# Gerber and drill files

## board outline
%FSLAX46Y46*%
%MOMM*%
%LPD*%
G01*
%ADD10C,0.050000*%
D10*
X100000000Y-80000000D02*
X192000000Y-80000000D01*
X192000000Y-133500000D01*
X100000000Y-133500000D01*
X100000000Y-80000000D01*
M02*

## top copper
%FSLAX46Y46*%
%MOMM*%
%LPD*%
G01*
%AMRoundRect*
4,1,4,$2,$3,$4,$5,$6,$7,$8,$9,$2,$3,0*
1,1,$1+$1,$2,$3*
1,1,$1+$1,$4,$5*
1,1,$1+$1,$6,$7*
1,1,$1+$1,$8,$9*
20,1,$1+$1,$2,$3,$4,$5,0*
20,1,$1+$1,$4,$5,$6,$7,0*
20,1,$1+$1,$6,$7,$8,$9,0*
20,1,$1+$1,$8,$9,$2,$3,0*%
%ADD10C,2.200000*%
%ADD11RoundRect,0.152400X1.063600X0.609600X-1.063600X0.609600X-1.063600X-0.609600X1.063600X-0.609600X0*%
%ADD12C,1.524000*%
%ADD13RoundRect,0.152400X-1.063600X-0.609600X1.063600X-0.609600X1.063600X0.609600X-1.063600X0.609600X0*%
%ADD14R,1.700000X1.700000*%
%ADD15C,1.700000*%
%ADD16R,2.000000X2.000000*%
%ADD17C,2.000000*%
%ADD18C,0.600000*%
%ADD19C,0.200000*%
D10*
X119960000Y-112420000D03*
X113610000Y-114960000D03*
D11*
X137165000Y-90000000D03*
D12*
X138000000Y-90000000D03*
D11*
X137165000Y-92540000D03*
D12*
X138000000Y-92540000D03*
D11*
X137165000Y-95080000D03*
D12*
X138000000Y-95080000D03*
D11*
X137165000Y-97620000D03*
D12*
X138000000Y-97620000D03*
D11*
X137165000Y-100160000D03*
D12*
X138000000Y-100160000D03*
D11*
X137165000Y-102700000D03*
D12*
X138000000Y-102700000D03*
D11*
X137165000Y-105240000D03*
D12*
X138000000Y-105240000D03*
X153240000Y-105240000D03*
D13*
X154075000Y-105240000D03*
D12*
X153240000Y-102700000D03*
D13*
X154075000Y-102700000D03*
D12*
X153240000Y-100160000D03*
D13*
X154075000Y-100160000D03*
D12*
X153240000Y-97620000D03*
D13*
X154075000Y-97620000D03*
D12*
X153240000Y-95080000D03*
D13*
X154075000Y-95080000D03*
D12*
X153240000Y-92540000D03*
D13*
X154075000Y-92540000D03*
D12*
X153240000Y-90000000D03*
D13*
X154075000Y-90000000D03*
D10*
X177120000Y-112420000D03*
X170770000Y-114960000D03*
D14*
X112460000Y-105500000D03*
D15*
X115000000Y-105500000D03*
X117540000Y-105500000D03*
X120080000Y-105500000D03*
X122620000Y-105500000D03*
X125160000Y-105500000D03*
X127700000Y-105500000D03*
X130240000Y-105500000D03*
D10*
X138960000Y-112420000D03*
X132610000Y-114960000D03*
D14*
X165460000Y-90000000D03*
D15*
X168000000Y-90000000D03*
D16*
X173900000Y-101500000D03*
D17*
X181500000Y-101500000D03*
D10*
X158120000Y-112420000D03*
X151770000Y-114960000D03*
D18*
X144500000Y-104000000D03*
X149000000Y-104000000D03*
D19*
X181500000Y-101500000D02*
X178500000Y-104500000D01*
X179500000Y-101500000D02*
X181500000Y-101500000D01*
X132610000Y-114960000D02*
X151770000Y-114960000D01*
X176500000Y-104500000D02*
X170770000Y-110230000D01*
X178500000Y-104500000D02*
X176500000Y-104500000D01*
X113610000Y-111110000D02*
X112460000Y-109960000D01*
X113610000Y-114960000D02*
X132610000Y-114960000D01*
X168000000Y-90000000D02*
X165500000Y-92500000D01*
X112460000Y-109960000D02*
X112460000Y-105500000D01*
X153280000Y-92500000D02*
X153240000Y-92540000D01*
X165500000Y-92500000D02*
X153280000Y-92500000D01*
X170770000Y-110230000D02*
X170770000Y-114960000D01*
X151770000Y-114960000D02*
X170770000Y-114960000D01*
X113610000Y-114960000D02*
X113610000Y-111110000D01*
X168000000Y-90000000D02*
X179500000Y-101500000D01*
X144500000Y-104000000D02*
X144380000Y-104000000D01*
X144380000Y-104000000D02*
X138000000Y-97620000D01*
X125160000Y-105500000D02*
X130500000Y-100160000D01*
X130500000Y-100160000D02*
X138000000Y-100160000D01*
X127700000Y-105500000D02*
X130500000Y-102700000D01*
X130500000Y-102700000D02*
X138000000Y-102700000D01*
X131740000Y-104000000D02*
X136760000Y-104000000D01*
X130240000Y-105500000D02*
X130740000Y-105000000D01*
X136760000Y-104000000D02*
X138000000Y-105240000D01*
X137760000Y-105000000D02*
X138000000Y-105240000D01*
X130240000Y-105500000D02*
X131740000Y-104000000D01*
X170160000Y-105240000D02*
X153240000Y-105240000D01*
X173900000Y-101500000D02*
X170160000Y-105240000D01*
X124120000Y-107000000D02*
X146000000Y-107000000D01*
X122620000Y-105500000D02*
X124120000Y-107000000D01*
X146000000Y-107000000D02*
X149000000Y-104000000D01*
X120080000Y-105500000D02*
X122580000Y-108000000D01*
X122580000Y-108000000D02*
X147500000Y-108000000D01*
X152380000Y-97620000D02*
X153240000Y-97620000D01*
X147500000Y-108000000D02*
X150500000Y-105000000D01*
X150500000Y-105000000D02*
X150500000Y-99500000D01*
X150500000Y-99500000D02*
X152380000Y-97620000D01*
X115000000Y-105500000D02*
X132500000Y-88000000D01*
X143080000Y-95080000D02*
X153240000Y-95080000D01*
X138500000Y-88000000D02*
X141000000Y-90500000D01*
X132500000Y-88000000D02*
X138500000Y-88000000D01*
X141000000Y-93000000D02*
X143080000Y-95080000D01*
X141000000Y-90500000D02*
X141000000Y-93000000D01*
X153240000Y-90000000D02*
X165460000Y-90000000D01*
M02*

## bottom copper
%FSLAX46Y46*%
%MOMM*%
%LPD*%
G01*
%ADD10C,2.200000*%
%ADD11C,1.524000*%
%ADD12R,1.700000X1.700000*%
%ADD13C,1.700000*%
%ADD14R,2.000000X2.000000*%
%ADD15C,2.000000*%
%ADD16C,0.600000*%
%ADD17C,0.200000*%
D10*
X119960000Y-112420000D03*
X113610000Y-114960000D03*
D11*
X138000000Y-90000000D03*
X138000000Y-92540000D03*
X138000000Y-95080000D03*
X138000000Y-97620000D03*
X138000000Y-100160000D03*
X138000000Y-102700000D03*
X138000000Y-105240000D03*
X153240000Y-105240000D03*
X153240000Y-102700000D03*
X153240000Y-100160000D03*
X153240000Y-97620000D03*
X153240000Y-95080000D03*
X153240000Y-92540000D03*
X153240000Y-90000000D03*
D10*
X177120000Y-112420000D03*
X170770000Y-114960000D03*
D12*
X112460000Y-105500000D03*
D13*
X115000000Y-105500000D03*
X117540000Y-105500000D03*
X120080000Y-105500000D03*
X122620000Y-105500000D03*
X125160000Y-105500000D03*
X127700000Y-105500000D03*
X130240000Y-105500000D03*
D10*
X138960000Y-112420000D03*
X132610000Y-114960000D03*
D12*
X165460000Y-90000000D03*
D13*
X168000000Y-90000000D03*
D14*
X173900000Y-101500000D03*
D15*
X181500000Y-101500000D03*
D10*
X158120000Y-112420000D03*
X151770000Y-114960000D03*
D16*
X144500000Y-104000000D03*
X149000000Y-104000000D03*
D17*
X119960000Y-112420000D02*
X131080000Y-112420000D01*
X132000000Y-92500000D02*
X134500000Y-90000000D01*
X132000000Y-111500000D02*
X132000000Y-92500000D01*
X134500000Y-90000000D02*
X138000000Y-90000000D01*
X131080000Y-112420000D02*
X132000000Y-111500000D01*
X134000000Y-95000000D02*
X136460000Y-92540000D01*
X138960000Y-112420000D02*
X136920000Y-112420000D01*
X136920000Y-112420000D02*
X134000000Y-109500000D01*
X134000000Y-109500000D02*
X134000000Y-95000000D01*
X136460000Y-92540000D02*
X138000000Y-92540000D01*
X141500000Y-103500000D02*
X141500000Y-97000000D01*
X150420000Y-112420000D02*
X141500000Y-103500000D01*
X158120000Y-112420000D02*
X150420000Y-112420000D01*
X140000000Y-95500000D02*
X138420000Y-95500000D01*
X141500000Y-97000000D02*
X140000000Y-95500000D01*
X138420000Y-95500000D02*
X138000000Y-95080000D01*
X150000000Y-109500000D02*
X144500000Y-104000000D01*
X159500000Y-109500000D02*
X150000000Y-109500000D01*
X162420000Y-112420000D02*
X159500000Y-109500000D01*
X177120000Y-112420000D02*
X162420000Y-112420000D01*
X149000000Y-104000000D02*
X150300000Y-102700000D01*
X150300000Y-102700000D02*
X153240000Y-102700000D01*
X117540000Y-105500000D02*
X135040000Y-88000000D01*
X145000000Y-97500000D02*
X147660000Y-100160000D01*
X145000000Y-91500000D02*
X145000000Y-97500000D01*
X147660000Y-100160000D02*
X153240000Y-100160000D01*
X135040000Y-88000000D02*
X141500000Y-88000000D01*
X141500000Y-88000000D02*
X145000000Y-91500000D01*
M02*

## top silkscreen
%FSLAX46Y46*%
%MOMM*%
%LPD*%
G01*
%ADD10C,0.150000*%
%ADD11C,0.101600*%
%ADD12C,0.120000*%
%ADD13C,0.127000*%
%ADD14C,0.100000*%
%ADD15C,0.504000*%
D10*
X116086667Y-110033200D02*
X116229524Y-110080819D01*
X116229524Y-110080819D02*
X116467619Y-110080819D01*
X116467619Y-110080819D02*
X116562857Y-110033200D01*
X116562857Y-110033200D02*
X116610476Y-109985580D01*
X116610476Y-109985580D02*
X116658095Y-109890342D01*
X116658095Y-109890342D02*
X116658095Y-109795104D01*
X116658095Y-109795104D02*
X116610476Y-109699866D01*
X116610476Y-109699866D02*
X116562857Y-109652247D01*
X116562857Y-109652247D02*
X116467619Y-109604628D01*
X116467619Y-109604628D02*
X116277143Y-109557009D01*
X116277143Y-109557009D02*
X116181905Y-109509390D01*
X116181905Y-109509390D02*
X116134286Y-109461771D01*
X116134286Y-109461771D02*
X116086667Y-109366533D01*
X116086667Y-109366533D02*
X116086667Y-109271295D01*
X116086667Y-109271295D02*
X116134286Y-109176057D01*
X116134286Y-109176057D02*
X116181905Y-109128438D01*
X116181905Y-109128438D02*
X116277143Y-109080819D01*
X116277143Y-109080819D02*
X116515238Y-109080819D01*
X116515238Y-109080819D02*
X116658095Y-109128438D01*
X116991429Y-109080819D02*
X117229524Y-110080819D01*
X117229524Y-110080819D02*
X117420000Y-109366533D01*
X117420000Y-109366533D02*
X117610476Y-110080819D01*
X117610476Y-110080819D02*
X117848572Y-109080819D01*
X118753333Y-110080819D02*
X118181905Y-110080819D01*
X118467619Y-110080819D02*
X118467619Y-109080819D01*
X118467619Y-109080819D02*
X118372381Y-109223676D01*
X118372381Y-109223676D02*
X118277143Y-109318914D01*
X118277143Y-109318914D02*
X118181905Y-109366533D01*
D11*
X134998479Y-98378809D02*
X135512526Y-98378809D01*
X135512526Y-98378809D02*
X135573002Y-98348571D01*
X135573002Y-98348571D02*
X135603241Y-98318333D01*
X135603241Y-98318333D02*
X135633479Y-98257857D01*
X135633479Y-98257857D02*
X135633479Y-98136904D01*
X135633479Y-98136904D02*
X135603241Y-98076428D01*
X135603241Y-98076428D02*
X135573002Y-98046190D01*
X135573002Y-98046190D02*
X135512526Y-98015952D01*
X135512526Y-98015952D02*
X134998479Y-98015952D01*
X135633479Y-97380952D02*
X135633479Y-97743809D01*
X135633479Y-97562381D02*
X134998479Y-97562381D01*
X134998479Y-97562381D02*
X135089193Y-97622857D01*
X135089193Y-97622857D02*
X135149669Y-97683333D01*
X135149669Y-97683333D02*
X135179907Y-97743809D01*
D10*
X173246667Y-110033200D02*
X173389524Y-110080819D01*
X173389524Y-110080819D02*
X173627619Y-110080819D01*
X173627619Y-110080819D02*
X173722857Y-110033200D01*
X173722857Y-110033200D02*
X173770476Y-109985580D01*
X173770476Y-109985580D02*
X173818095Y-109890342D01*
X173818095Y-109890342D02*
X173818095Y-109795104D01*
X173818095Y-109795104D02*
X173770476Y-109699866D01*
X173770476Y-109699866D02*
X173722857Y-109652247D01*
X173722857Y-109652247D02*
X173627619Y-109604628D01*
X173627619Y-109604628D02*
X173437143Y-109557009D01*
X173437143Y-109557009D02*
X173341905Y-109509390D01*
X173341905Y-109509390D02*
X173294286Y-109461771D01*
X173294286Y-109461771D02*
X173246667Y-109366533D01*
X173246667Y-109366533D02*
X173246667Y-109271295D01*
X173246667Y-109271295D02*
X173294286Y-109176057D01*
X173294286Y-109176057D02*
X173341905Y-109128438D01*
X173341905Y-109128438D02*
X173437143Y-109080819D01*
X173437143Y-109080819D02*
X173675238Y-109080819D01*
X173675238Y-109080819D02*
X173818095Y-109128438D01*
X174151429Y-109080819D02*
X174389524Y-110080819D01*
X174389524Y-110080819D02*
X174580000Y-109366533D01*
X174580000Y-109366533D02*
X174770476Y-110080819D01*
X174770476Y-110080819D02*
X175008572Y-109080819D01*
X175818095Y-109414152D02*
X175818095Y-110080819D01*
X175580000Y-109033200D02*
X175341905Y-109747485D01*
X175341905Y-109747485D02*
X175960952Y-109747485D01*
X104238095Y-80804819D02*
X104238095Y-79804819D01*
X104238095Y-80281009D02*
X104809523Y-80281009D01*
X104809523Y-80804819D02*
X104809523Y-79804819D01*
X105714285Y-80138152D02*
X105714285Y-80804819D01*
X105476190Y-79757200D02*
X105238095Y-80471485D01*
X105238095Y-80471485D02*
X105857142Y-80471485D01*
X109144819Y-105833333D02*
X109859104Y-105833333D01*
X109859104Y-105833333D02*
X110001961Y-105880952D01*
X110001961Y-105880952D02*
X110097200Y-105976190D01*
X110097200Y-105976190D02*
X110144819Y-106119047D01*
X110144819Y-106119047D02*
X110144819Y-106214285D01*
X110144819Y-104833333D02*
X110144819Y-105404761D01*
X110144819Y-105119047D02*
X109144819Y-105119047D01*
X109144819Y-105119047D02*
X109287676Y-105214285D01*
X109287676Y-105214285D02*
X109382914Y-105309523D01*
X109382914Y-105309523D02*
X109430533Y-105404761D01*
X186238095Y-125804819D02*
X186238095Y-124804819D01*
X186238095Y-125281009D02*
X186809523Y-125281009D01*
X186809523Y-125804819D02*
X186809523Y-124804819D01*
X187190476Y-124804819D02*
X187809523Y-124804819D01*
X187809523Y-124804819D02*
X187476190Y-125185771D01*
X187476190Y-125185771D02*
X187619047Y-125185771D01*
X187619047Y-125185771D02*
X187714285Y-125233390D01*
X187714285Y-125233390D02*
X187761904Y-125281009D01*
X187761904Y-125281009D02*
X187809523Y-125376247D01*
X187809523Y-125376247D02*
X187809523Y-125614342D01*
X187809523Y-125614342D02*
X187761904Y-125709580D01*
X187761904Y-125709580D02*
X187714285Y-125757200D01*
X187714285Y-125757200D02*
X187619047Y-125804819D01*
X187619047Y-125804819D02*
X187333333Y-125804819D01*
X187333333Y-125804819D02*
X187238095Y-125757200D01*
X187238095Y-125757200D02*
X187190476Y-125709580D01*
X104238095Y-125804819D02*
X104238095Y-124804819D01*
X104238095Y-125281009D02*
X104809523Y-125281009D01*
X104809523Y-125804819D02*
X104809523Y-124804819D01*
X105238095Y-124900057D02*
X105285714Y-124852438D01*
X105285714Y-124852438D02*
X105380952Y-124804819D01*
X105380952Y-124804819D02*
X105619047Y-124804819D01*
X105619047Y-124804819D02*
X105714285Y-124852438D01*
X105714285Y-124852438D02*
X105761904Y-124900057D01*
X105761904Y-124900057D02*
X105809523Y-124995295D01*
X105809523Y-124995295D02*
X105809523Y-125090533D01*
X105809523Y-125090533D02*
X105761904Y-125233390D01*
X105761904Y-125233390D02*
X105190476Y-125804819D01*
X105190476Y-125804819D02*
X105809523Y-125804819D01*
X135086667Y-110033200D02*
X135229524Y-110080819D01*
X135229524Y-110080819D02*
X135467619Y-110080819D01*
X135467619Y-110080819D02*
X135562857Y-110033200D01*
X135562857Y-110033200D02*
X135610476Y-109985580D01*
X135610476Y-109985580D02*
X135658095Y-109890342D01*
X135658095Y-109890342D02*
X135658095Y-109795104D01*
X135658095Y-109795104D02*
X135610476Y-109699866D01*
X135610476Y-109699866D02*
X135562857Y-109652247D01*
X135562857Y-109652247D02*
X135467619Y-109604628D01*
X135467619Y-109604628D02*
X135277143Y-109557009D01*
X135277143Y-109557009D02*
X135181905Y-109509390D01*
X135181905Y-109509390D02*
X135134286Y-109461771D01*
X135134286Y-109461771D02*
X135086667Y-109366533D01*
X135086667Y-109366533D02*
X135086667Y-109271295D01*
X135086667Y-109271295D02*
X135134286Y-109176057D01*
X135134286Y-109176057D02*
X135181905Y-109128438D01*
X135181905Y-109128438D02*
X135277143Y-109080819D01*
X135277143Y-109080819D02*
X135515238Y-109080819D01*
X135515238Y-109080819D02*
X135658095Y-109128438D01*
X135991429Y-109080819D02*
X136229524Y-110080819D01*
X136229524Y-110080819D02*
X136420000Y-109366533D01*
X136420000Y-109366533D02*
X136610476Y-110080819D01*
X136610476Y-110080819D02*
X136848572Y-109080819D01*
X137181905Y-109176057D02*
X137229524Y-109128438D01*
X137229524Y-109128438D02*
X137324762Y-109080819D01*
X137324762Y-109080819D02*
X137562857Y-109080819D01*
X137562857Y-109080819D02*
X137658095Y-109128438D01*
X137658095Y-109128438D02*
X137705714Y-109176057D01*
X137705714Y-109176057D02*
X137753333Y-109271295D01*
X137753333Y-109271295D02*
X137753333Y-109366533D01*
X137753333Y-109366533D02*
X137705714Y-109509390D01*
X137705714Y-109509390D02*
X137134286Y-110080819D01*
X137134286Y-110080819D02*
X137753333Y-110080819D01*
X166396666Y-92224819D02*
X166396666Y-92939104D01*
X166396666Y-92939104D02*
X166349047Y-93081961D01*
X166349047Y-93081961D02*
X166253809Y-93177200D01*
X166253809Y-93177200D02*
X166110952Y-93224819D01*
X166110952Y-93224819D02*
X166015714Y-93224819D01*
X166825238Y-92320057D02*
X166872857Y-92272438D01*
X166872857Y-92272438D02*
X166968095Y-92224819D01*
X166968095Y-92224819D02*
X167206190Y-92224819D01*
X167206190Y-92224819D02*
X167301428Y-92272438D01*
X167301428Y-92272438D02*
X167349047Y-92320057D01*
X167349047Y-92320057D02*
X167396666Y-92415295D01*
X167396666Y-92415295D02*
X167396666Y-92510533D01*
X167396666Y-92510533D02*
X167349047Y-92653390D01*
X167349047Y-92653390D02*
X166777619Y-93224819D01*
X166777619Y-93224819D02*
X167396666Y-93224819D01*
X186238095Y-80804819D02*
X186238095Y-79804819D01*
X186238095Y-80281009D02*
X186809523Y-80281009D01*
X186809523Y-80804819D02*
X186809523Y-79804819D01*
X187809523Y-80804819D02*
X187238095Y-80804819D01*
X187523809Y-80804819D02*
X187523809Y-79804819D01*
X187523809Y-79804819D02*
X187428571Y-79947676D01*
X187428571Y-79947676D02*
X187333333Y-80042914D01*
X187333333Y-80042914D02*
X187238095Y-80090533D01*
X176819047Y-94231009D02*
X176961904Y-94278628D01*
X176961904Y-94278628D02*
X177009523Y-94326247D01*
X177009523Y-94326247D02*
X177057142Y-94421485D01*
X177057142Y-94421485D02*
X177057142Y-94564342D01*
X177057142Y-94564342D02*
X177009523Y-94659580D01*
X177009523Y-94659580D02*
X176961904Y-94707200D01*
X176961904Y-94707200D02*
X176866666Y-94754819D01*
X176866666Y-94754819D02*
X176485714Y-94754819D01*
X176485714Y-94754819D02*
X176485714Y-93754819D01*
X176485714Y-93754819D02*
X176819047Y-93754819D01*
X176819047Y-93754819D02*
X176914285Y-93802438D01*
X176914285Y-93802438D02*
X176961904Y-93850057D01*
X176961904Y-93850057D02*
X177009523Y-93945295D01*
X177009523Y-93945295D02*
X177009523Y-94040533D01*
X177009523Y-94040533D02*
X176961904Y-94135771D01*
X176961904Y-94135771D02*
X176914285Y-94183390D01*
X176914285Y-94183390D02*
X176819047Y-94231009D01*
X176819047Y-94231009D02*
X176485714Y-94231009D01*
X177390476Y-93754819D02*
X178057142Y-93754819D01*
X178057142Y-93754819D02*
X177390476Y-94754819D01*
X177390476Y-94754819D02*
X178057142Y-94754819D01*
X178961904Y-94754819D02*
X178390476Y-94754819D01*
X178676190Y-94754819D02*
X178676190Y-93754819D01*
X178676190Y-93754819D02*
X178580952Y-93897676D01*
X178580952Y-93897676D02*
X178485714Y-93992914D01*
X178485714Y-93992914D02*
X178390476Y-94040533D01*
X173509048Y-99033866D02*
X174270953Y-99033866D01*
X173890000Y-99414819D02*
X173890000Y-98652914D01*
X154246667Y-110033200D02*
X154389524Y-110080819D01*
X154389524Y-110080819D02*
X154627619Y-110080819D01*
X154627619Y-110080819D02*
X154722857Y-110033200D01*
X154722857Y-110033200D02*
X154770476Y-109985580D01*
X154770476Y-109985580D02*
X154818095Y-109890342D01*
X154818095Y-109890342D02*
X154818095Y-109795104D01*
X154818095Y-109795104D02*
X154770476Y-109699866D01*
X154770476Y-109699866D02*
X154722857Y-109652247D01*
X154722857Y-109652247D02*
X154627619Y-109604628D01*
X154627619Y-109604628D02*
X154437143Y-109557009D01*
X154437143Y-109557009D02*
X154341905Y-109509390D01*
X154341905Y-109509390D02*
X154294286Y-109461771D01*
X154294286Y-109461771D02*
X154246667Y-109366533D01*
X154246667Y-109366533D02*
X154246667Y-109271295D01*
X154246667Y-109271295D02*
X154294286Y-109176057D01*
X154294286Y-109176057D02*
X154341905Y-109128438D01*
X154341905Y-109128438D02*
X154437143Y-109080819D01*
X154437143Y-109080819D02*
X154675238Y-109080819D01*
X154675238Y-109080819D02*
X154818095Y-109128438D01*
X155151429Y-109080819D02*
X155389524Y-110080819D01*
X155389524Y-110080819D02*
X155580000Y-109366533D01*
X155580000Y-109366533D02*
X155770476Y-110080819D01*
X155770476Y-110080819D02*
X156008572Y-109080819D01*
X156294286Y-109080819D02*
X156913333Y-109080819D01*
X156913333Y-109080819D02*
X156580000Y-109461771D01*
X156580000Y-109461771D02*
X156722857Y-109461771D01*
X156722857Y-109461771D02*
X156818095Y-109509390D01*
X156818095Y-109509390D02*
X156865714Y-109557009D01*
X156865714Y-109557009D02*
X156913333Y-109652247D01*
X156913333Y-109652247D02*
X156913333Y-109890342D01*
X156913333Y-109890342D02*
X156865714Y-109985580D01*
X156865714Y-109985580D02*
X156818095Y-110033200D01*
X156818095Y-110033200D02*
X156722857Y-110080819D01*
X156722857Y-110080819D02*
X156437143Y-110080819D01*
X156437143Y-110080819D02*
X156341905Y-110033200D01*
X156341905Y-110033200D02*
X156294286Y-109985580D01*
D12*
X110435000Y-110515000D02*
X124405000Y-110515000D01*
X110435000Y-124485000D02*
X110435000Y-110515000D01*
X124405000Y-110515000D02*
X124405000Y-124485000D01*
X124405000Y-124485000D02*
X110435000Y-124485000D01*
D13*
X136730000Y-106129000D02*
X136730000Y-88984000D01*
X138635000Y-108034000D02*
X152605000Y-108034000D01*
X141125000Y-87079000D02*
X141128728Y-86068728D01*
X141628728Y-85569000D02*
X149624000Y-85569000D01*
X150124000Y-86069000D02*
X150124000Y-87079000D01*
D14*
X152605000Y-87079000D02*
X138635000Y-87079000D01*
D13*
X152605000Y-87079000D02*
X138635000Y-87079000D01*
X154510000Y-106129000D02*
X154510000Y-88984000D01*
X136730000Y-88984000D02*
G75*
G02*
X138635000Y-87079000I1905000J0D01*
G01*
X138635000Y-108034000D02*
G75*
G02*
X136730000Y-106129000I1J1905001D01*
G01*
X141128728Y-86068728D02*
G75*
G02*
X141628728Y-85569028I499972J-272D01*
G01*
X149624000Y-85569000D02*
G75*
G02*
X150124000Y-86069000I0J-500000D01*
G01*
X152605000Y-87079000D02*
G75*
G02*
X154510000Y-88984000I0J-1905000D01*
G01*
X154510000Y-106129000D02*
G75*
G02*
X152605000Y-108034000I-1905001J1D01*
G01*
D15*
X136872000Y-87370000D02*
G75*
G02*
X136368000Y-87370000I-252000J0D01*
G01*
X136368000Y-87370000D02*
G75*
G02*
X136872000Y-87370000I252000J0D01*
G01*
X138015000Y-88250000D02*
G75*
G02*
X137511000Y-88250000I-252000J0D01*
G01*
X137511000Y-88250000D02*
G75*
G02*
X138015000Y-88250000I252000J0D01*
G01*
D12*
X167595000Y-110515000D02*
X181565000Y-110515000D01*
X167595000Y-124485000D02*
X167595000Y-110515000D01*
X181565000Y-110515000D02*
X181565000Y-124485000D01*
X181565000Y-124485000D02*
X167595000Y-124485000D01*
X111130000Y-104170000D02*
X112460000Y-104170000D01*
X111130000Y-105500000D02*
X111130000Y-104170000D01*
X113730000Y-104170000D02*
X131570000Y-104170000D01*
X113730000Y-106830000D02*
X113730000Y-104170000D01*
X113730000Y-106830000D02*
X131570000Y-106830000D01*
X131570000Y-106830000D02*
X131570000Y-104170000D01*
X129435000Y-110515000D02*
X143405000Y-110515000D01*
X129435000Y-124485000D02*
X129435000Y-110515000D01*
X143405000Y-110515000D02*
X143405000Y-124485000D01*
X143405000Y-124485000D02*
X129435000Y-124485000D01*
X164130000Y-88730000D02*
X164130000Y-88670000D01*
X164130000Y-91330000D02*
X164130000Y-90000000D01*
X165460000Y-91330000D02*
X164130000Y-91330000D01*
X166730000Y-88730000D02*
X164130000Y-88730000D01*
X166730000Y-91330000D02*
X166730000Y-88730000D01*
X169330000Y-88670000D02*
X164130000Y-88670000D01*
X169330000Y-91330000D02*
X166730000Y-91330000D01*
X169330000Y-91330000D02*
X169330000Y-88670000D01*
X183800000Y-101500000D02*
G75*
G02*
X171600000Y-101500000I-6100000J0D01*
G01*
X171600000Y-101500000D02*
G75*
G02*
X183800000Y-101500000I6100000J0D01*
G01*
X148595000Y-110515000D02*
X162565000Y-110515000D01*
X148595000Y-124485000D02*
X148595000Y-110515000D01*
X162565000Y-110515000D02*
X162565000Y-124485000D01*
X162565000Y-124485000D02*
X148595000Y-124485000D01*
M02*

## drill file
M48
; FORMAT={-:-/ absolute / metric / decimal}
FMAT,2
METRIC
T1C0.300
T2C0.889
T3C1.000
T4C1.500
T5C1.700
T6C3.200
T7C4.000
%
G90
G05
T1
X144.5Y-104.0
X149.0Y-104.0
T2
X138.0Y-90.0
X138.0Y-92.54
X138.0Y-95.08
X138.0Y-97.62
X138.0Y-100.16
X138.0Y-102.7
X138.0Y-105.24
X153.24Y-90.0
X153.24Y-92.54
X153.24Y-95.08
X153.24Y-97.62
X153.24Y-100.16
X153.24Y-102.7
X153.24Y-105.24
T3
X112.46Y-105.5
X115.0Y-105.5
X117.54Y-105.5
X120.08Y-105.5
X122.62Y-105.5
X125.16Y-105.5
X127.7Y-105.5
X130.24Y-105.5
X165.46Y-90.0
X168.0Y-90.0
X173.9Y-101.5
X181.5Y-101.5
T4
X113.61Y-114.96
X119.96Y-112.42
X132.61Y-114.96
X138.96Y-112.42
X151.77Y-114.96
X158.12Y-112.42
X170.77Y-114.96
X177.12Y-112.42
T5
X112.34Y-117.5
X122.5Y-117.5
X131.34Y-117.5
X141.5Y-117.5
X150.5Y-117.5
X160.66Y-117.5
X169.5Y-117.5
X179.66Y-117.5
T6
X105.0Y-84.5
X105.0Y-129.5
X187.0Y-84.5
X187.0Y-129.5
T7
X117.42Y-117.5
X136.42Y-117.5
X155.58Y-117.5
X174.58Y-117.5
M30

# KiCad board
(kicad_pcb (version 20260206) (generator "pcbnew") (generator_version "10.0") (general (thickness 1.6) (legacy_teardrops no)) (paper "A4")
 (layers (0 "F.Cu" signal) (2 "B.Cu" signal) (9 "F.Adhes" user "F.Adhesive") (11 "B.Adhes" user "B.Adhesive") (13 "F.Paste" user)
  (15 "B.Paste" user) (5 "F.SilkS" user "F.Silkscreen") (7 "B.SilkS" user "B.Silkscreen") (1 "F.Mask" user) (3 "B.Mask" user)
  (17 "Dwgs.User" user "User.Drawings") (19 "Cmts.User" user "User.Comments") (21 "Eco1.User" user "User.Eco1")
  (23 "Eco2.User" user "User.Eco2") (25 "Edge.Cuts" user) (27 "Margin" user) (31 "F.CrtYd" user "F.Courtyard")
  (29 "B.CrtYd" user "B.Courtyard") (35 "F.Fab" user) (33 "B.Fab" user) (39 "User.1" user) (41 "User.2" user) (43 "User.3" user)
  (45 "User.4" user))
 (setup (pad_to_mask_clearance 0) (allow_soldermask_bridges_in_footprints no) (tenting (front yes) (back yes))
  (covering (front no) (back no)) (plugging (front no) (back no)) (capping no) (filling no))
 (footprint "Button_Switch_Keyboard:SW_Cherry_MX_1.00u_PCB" (layer "F.Cu") (at 119.96 112.42)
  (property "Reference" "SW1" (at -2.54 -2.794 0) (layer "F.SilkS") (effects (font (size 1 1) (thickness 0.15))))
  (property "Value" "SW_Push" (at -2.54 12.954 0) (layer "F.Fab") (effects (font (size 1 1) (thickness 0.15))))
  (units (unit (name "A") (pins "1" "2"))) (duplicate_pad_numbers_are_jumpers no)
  (fp_line (start -9.525 -1.905) (end 4.445 -1.905) (stroke (width 0.12) (type solid)) (layer "F.SilkS"))
  (fp_line (start -9.525 12.065) (end -9.525 -1.905) (stroke (width 0.12) (type solid)) (layer "F.SilkS"))
  (fp_line (start 4.445 -1.905) (end 4.445 12.065) (stroke (width 0.12) (type solid)) (layer "F.SilkS"))
  (fp_line (start 4.445 12.065) (end -9.525 12.065) (stroke (width 0.12) (type solid)) (layer "F.SilkS"))
  (pad "" np_thru_hole circle (at -7.62 5.08) (size 1.7 1.7) (drill 1.7) (layers "*.Cu" "*.Mask"))
  (pad "" np_thru_hole circle (at -2.54 5.08) (size 4 4) (drill 4) (layers "*.Cu" "*.Mask"))
  (pad "" np_thru_hole circle (at 2.54 5.08) (size 1.7 1.7) (drill 1.7) (layers "*.Cu" "*.Mask"))
  (pad "1" thru_hole circle (at 0 0) (size 2.2 2.2) (drill 1.5) (layers "*.Cu" "*.Mask") (remove_unused_layers no) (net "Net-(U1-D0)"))
  (pad "2" thru_hole circle (at -6.35 2.54) (size 2.2 2.2) (drill 1.5) (layers "*.Cu" "*.Mask") (remove_unused_layers no) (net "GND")))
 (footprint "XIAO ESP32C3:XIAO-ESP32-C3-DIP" (layer "F.Cu") (at 145.62 97.62 90)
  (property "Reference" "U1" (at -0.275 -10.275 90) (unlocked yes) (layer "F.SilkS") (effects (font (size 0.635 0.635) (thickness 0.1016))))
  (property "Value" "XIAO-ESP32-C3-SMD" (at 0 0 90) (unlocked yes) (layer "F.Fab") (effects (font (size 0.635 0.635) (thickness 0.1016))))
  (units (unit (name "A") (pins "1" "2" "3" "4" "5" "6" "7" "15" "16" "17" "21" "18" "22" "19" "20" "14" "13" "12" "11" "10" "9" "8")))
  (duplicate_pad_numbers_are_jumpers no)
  (fp_line (start -8.509 -8.89) (end 8.636 -8.89) (stroke (width 0.127) (type solid)) (layer "F.SilkS"))
  (fp_line (start -10.414 -6.985) (end -10.414 6.985) (stroke (width 0.127) (type solid)) (layer "F.SilkS"))
  (fp_line (start 10.541 -4.495) (end 11.551272 -4.491272) (stroke (width 0.127) (type solid)) (layer "F.SilkS"))
  (fp_line (start 12.051 -3.991272) (end 12.051 4.004) (stroke (width 0.127) (type solid)) (layer "F.SilkS"))
  (fp_line (start 11.551 4.504) (end 10.541 4.504) (stroke (width 0.127) (type solid)) (layer "F.SilkS"))
  (fp_line (start 10.541 6.985) (end 10.541 -6.985) (stroke (width 0.1) (type solid)) (layer "F.SilkS"))
  (fp_line (start 10.541 6.985) (end 10.541 -6.985) (stroke (width 0.127) (type solid)) (layer "F.SilkS"))
  (fp_line (start -8.509 8.89) (end 8.636 8.89) (stroke (width 0.127) (type solid)) (layer "F.SilkS"))
  (fp_arc (start 8.636 -8.89) (mid 9.983038 -8.332038) (end 10.541 -6.985) (stroke (width 0.127) (type solid)) (layer "F.SilkS"))
  (fp_arc (start -10.414 -6.985) (mid -9.856038 -8.332038) (end -8.509 -8.89) (stroke (width 0.127) (type solid)) (layer "F.SilkS"))
  (fp_arc (start 11.551272 -4.491272) (mid 11.904644 -4.344724) (end 12.051 -3.991272) (stroke (width 0.127) (type default))
   (layer "F.SilkS"))
  (fp_arc (start 12.051 4.004) (mid 11.904553 4.357553) (end 11.551 4.504) (stroke (width 0.127) (type default)) (layer "F.SilkS"))
  (fp_arc (start 10.541 6.985) (mid 9.983038 8.332038) (end 8.636 8.89) (stroke (width 0.127) (type solid)) (layer "F.SilkS"))
  (fp_arc (start -8.509 8.89) (mid -9.856038 8.332038) (end -10.414 6.985) (stroke (width 0.127) (type solid)) (layer "F.SilkS"))
  (fp_circle (center 10.25 -9) (end 10.504 -9) (stroke (width 0.5) (type solid)) (fill yes) (layer "F.SilkS"))
  (fp_circle (center 9.37 -7.857) (end 9.624 -7.857) (stroke (width 0.5) (type solid)) (fill yes) (layer "F.SilkS"))
  (pad "1" smd roundrect (at 7.62 -8.455 180) (size 2.432 1.524) (layers "F.Cu" "F.Mask") (roundrect_rratio 0.1) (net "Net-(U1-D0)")
   (thermal_bridge_angle 45))
  (pad "1" thru_hole circle (at 7.62 -7.62 180) (size 1.524 1.524) (drill 0.889) (layers "*.Cu" "*.Mask") (remove_unused_layers no)
   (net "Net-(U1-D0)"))
  (pad "2" smd roundrect (at 5.08 -8.455 180) (size 2.432 1.524) (layers "F.Cu" "F.Mask") (roundrect_rratio 0.1) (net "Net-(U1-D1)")
   (thermal_bridge_angle 45))
  (pad "2" thru_hole circle (at 5.08 -7.62 180) (size 1.524 1.524) (drill 0.889) (layers "*.Cu" "*.Mask") (remove_unused_layers no)
   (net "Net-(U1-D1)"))
  (pad "3" smd roundrect (at 2.54 -8.455 180) (size 2.432 1.524) (layers "F.Cu" "F.Mask") (roundrect_rratio 0.1) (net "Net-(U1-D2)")
   (thermal_bridge_angle 45))
  (pad "3" thru_hole circle (at 2.54 -7.62 180) (size 1.524 1.524) (drill 0.889) (layers "*.Cu" "*.Mask") (remove_unused_layers no)
   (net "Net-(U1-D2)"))
  (pad "4" smd roundrect (at 0 -8.455 180) (size 2.432 1.524) (layers "F.Cu" "F.Mask") (roundrect_rratio 0.1) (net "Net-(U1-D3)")
   (thermal_bridge_angle 45))
  (pad "4" thru_hole circle (at 0 -7.62 180) (size 1.524 1.524) (drill 0.889) (layers "*.Cu" "*.Mask") (remove_unused_layers no)
   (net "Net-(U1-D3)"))
  (pad "5" smd roundrect (at -2.54 -8.455 180) (size 2.432 1.524) (layers "F.Cu" "F.Mask") (roundrect_rratio 0.1) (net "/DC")
   (thermal_bridge_angle 45))
  (pad "5" thru_hole circle (at -2.54 -7.62 180) (size 1.524 1.524) (drill 0.889) (layers "*.Cu" "*.Mask") (remove_unused_layers no)
   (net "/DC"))
  (pad "6" smd roundrect (at -5.08 -8.455 180) (size 2.432 1.524) (layers "F.Cu" "F.Mask") (roundrect_rratio 0.1) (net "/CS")
   (thermal_bridge_angle 45))
  (pad "6" thru_hole circle (at -5.08 -7.62 180) (size 1.524 1.524) (drill 0.889) (layers "*.Cu" "*.Mask") (remove_unused_layers no)
   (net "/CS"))
  (pad "7" smd roundrect (at -7.62 -8.455 180) (size 2.432 1.524) (layers "F.Cu" "F.Mask") (roundrect_rratio 0.1) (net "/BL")
   (thermal_bridge_angle 45))
  (pad "7" thru_hole circle (at -7.62 -7.62 180) (size 1.524 1.524) (drill 0.889) (layers "*.Cu" "*.Mask") (remove_unused_layers no)
   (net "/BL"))
  (pad "8" thru_hole circle (at -7.62 7.62) (size 1.524 1.524) (drill 0.889) (layers "*.Cu" "*.Mask") (remove_unused_layers no)
   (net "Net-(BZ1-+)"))
  (pad "8" smd roundrect (at -7.62 8.455) (size 2.432 1.524) (layers "F.Cu" "F.Mask") (roundrect_rratio 0.1) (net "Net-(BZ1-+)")
   (thermal_bridge_angle 45))
  (pad "9" thru_hole circle (at -5.08 7.62) (size 1.524 1.524) (drill 0.889) (layers "*.Cu" "*.Mask") (remove_unused_layers no) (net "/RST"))
  (pad "9" smd roundrect (at -5.08 8.455) (size 2.432 1.524) (layers "F.Cu" "F.Mask") (roundrect_rratio 0.1) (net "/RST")
   (thermal_bridge_angle 45))
  (pad "10" thru_hole circle (at -2.54 7.62) (size 1.524 1.524) (drill 0.889) (layers "*.Cu" "*.Mask") (remove_unused_layers no)
   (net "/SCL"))
  (pad "10" smd roundrect (at -2.54 8.455) (size 2.432 1.524) (layers "F.Cu" "F.Mask") (roundrect_rratio 0.1) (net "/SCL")
   (thermal_bridge_angle 45))
  (pad "11" thru_hole circle (at 0 7.62) (size 1.524 1.524) (drill 0.889) (layers "*.Cu" "*.Mask") (remove_unused_layers no) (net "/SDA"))
  (pad "11" smd roundrect (at 0 8.455) (size 2.432 1.524) (layers "F.Cu" "F.Mask") (roundrect_rratio 0.1) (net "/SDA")
   (thermal_bridge_angle 45))
  (pad "12" thru_hole circle (at 2.54 7.62) (size 1.524 1.524) (drill 0.889) (layers "*.Cu" "*.Mask") (remove_unused_layers no) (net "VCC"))
  (pad "12" smd roundrect (at 2.54 8.455) (size 2.432 1.524) (layers "F.Cu" "F.Mask") (roundrect_rratio 0.1) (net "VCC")
   (thermal_bridge_angle 45))
  (pad "13" thru_hole circle (at 5.08 7.62) (size 1.524 1.524) (drill 0.889) (layers "*.Cu" "*.Mask") (remove_unused_layers no) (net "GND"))
  (pad "13" smd roundrect (at 5.08 8.455) (size 2.432 1.524) (layers "F.Cu" "F.Mask") (roundrect_rratio 0.1) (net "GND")
   (thermal_bridge_angle 45))
  (pad "14" thru_hole circle (at 7.62 7.62) (size 1.524 1.524) (drill 0.889) (layers "*.Cu" "*.Mask") (remove_unused_layers no)
   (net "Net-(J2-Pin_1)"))
  (pad "14" smd roundrect (at 7.62 8.455) (size 2.432 1.524) (layers "F.Cu" "F.Mask") (roundrect_rratio 0.1) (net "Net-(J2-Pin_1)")
   (thermal_bridge_angle 45)))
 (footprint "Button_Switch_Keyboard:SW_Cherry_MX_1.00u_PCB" (layer "F.Cu") (at 177.12 112.42)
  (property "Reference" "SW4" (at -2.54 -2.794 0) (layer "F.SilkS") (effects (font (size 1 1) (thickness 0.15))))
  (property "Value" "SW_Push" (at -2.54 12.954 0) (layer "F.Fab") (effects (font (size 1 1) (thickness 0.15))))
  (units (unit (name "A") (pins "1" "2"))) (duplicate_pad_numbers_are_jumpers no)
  (fp_line (start -9.525 -1.905) (end 4.445 -1.905) (stroke (width 0.12) (type solid)) (layer "F.SilkS"))
  (fp_line (start -9.525 12.065) (end -9.525 -1.905) (stroke (width 0.12) (type solid)) (layer "F.SilkS"))
  (fp_line (start 4.445 -1.905) (end 4.445 12.065) (stroke (width 0.12) (type solid)) (layer "F.SilkS"))
  (fp_line (start 4.445 12.065) (end -9.525 12.065) (stroke (width 0.12) (type solid)) (layer "F.SilkS"))
  (pad "" np_thru_hole circle (at -7.62 5.08) (size 1.7 1.7) (drill 1.7) (layers "*.Cu" "*.Mask"))
  (pad "" np_thru_hole circle (at -2.54 5.08) (size 4 4) (drill 4) (layers "*.Cu" "*.Mask"))
  (pad "" np_thru_hole circle (at 2.54 5.08) (size 1.7 1.7) (drill 1.7) (layers "*.Cu" "*.Mask"))
  (pad "1" thru_hole circle (at 0 0) (size 2.2 2.2) (drill 1.5) (layers "*.Cu" "*.Mask") (remove_unused_layers no) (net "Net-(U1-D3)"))
  (pad "2" thru_hole circle (at -6.35 2.54) (size 2.2 2.2) (drill 1.5) (layers "*.Cu" "*.Mask") (remove_unused_layers no) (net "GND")))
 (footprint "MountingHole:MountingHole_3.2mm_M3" (layer "F.Cu") (at 105 84.5)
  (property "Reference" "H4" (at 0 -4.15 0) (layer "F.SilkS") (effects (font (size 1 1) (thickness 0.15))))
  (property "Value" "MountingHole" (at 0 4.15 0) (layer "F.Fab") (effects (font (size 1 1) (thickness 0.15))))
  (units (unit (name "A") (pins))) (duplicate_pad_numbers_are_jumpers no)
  (pad "" np_thru_hole circle (at 0 0) (size 3.2 3.2) (drill 3.2) (layers "*.Cu" "*.Mask")))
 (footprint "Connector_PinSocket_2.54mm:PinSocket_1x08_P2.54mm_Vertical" (layer "F.Cu") (at 112.46 105.5 90)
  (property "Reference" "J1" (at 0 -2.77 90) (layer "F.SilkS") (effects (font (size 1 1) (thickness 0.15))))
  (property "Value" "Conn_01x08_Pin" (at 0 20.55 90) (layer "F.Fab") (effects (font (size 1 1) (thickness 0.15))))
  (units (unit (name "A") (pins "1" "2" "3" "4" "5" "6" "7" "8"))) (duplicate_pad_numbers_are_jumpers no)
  (fp_line (start 1.33 -1.33) (end 1.33 0) (stroke (width 0.12) (type solid)) (layer "F.SilkS"))
  (fp_line (start 0 -1.33) (end 1.33 -1.33) (stroke (width 0.12) (type solid)) (layer "F.SilkS"))
  (fp_line (start 1.33 1.27) (end 1.33 19.11) (stroke (width 0.12) (type solid)) (layer "F.SilkS"))
  (fp_line (start -1.33 1.27) (end 1.33 1.27) (stroke (width 0.12) (type solid)) (layer "F.SilkS"))
  (fp_line (start -1.33 1.27) (end -1.33 19.11) (stroke (width 0.12) (type solid)) (layer "F.SilkS"))
  (fp_line (start -1.33 19.11) (end 1.33 19.11) (stroke (width 0.12) (type solid)) (layer "F.SilkS"))
  (pad "1" thru_hole rect (at 0 0 90) (size 1.7 1.7) (drill 1) (layers "*.Cu" "*.Mask") (remove_unused_layers no) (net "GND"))
  (pad "2" thru_hole circle (at 0 2.54 90) (size 1.7 1.7) (drill 1) (layers "*.Cu" "*.Mask") (remove_unused_layers no) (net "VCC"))
  (pad "3" thru_hole circle (at 0 5.08 90) (size 1.7 1.7) (drill 1) (layers "*.Cu" "*.Mask") (remove_unused_layers no) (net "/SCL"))
  (pad "4" thru_hole circle (at 0 7.62 90) (size 1.7 1.7) (drill 1) (layers "*.Cu" "*.Mask") (remove_unused_layers no) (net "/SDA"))
  (pad "5" thru_hole circle (at 0 10.16 90) (size 1.7 1.7) (drill 1) (layers "*.Cu" "*.Mask") (remove_unused_layers no) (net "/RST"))
  (pad "6" thru_hole circle (at 0 12.7 90) (size 1.7 1.7) (drill 1) (layers "*.Cu" "*.Mask") (remove_unused_layers no) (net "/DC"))
  (pad "7" thru_hole circle (at 0 15.24 90) (size 1.7 1.7) (drill 1) (layers "*.Cu" "*.Mask") (remove_unused_layers no) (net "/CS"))
  (pad "8" thru_hole circle (at 0 17.78 90) (size 1.7 1.7) (drill 1) (layers "*.Cu" "*.Mask") (remove_unused_layers no) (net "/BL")))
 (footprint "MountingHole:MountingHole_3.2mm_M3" (layer "F.Cu") (at 187 129.5)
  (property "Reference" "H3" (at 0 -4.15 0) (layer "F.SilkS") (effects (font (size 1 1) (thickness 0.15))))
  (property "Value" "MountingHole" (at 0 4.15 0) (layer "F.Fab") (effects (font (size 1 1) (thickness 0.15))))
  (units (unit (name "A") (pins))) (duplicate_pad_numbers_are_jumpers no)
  (pad "" np_thru_hole circle (at 0 0) (size 3.2 3.2) (drill 3.2) (layers "*.Cu" "*.Mask")))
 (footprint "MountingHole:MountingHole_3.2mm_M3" (layer "F.Cu") (at 105 129.5)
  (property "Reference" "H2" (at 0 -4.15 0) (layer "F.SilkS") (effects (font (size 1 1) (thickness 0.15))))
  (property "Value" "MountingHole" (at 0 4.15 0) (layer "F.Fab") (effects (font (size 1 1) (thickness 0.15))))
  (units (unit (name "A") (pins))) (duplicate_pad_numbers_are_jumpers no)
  (pad "" np_thru_hole circle (at 0 0) (size 3.2 3.2) (drill 3.2) (layers "*.Cu" "*.Mask")))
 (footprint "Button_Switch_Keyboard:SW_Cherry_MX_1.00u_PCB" (layer "F.Cu") (at 138.96 112.42)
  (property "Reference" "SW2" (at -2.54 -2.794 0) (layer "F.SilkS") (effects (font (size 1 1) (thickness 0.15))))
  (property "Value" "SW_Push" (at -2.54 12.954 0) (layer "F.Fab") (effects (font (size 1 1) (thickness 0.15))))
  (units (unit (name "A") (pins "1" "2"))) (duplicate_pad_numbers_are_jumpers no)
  (fp_line (start -9.525 -1.905) (end 4.445 -1.905) (stroke (width 0.12) (type solid)) (layer "F.SilkS"))
  (fp_line (start -9.525 12.065) (end -9.525 -1.905) (stroke (width 0.12) (type solid)) (layer "F.SilkS"))
  (fp_line (start 4.445 -1.905) (end 4.445 12.065) (stroke (width 0.12) (type solid)) (layer "F.SilkS"))
  (fp_line (start 4.445 12.065) (end -9.525 12.065) (stroke (width 0.12) (type solid)) (layer "F.SilkS"))
  (pad "" np_thru_hole circle (at -7.62 5.08) (size 1.7 1.7) (drill 1.7) (layers "*.Cu" "*.Mask"))
  (pad "" np_thru_hole circle (at -2.54 5.08) (size 4 4) (drill 4) (layers "*.Cu" "*.Mask"))
  (pad "" np_thru_hole circle (at 2.54 5.08) (size 1.7 1.7) (drill 1.7) (layers "*.Cu" "*.Mask"))
  (pad "1" thru_hole circle (at 0 0) (size 2.2 2.2) (drill 1.5) (layers "*.Cu" "*.Mask") (remove_unused_layers no) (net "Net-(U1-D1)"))
  (pad "2" thru_hole circle (at -6.35 2.54) (size 2.2 2.2) (drill 1.5) (layers "*.Cu" "*.Mask") (remove_unused_layers no) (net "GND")))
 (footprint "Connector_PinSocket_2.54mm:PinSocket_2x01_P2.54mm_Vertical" (layer "F.Cu") (at 165.46 90 180)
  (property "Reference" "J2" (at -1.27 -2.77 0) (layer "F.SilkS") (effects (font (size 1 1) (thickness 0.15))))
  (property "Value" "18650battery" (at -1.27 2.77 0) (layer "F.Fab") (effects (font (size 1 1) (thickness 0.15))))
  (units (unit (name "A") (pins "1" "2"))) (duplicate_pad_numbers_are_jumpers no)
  (fp_line (start 1.33 1.27) (end 1.33 1.33) (stroke (width 0.12) (type solid)) (layer "F.SilkS"))
  (fp_line (start 1.33 -1.33) (end 1.33 0) (stroke (width 0.12) (type solid)) (layer "F.SilkS"))
  (fp_line (start 0 -1.33) (end 1.33 -1.33) (stroke (width 0.12) (type solid)) (layer "F.SilkS"))
  (fp_line (start -1.27 1.27) (end 1.33 1.27) (stroke (width 0.12) (type solid)) (layer "F.SilkS"))
  (fp_line (start -1.27 -1.33) (end -1.27 1.27) (stroke (width 0.12) (type solid)) (layer "F.SilkS"))
  (fp_line (start -3.87 1.33) (end 1.33 1.33) (stroke (width 0.12) (type solid)) (layer "F.SilkS"))
  (fp_line (start -3.87 -1.33) (end -1.27 -1.33) (stroke (width 0.12) (type solid)) (layer "F.SilkS"))
  (fp_line (start -3.87 -1.33) (end -3.87 1.33) (stroke (width 0.12) (type solid)) (layer "F.SilkS"))
  (pad "1" thru_hole rect (at 0 0 180) (size 1.7 1.7) (drill 1) (layers "*.Cu" "*.Mask") (remove_unused_layers no) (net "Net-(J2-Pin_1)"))
  (pad "2" thru_hole circle (at -2.54 0 180) (size 1.7 1.7) (drill 1) (layers "*.Cu" "*.Mask") (remove_unused_layers no) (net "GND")))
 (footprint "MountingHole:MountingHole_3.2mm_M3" (layer "F.Cu") (at 187 84.5)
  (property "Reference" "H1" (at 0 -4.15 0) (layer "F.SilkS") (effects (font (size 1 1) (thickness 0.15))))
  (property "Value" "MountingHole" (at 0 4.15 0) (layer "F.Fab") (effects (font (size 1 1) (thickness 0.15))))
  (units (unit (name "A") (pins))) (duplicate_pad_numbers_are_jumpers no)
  (pad "" np_thru_hole circle (at 0 0) (size 3.2 3.2) (drill 3.2) (layers "*.Cu" "*.Mask")))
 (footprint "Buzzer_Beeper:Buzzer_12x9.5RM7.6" (layer "F.Cu") (at 173.9 101.5)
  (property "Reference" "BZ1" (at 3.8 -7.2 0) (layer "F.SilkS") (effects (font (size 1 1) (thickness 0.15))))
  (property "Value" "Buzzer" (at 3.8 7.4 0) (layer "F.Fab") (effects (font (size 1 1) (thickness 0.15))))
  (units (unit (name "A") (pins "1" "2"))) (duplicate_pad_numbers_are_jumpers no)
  (fp_circle (center 3.8 0) (end 9.9 0) (stroke (width 0.12) (type solid)) (fill no) (layer "F.SilkS"))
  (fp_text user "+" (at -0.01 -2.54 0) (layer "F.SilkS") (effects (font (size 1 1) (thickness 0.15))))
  (pad "1" thru_hole rect (at 0 0) (size 2 2) (drill 1) (layers "*.Cu" "*.Mask") (remove_unused_layers no) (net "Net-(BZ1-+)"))
  (pad "2" thru_hole circle (at 7.6 0) (size 2 2) (drill 1) (layers "*.Cu" "*.Mask") (remove_unused_layers no) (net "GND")))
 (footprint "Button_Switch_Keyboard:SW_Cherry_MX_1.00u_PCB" (layer "F.Cu") (at 158.12 112.42)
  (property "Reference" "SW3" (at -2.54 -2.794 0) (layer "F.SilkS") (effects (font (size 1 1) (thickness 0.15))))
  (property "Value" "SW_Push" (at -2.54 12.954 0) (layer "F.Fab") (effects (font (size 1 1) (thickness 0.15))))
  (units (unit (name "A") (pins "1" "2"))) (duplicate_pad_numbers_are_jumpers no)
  (fp_line (start -9.525 -1.905) (end 4.445 -1.905) (stroke (width 0.12) (type solid)) (layer "F.SilkS"))
  (fp_line (start -9.525 12.065) (end -9.525 -1.905) (stroke (width 0.12) (type solid)) (layer "F.SilkS"))
  (fp_line (start 4.445 -1.905) (end 4.445 12.065) (stroke (width 0.12) (type solid)) (layer "F.SilkS"))
  (fp_line (start 4.445 12.065) (end -9.525 12.065) (stroke (width 0.12) (type solid)) (layer "F.SilkS"))
  (pad "" np_thru_hole circle (at -7.62 5.08) (size 1.7 1.7) (drill 1.7) (layers "*.Cu" "*.Mask"))
  (pad "" np_thru_hole circle (at -2.54 5.08) (size 4 4) (drill 4) (layers "*.Cu" "*.Mask"))
  (pad "" np_thru_hole circle (at 2.54 5.08) (size 1.7 1.7) (drill 1.7) (layers "*.Cu" "*.Mask"))
  (pad "1" thru_hole circle (at 0 0) (size 2.2 2.2) (drill 1.5) (layers "*.Cu" "*.Mask") (remove_unused_layers no) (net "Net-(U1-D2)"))
  (pad "2" thru_hole circle (at -6.35 2.54) (size 2.2 2.2) (drill 1.5) (layers "*.Cu" "*.Mask") (remove_unused_layers no) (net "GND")))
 (gr_rect (start 100 80) (end 192 133.5) (stroke (width 0.05) (type default)) (fill no) (layer "Edge.Cuts"))
 (segment (start 119.96 112.42) (end 131.08 112.42) (width 0.2) (layer "B.Cu") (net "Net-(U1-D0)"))
 (segment (start 132 92.5) (end 134.5 90) (width 0.2) (layer "B.Cu") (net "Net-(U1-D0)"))
 (segment (start 132 111.5) (end 132 92.5) (width 0.2) (layer "B.Cu") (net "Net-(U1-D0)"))
 (segment (start 134.5 90) (end 138 90) (width 0.2) (layer "B.Cu") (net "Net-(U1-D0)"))
 (segment (start 131.08 112.42) (end 132 111.5) (width 0.2) (layer "B.Cu") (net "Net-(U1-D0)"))
 (segment (start 181.5 101.5) (end 178.5 104.5) (width 0.2) (layer "F.Cu") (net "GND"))
 (segment (start 179.5 101.5) (end 181.5 101.5) (width 0.2) (layer "F.Cu") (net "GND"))
 (segment (start 132.61 114.96) (end 151.77 114.96) (width 0.2) (layer "F.Cu") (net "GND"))
 (segment (start 176.5 104.5) (end 170.77 110.23) (width 0.2) (layer "F.Cu") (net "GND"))
 (segment (start 178.5 104.5) (end 176.5 104.5) (width 0.2) (layer "F.Cu") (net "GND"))
 (segment (start 113.61 111.11) (end 112.46 109.96) (width 0.2) (layer "F.Cu") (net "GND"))
 (segment (start 113.61 114.96) (end 132.61 114.96) (width 0.2) (layer "F.Cu") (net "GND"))
 (segment (start 168 90) (end 165.5 92.5) (width 0.2) (layer "F.Cu") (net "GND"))
 (segment (start 112.46 109.96) (end 112.46 105.5) (width 0.2) (layer "F.Cu") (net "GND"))
 (segment (start 153.28 92.5) (end 153.24 92.54) (width 0.2) (layer "F.Cu") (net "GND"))
 (segment (start 165.5 92.5) (end 153.28 92.5) (width 0.2) (layer "F.Cu") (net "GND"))
 (segment (start 170.77 110.23) (end 170.77 114.96) (width 0.2) (layer "F.Cu") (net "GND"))
 (segment (start 151.77 114.96) (end 170.77 114.96) (width 0.2) (layer "F.Cu") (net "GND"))
 (segment (start 113.61 114.96) (end 113.61 111.11) (width 0.2) (layer "F.Cu") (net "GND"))
 (segment (start 168 90) (end 179.5 101.5) (width 0.2) (layer "F.Cu") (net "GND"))
 (segment (start 134 95) (end 136.46 92.54) (width 0.2) (layer "B.Cu") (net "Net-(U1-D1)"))
 (segment (start 138.96 112.42) (end 136.92 112.42) (width 0.2) (layer "B.Cu") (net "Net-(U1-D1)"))
 (segment (start 136.92 112.42) (end 134 109.5) (width 0.2) (layer "B.Cu") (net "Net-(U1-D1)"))
 (segment (start 134 109.5) (end 134 95) (width 0.2) (layer "B.Cu") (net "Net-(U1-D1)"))
 (segment (start 136.46 92.54) (end 138 92.54) (width 0.2) (layer "B.Cu") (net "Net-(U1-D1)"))
 (segment (start 141.5 103.5) (end 141.5 97) (width 0.2) (layer "B.Cu") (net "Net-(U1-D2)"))
 (segment (start 150.42 112.42) (end 141.5 103.5) (width 0.2) (layer "B.Cu") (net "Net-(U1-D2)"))
 (segment (start 158.12 112.42) (end 150.42 112.42) (width 0.2) (layer "B.Cu") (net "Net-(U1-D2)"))
 (segment (start 140 95.5) (end 138.42 95.5) (width 0.2) (layer "B.Cu") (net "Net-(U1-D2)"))
 (segment (start 141.5 97) (end 140 95.5) (width 0.2) (layer "B.Cu") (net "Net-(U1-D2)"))
 (segment (start 138.42 95.5) (end 138 95.08) (width 0.2) (layer "B.Cu") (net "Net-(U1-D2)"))
 (segment (start 144.5 104) (end 144.38 104) (width 0.2) (layer "F.Cu") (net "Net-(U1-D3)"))
 (segment (start 144.38 104) (end 138 97.62) (width 0.2) (layer "F.Cu") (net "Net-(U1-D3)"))
 (via (at 144.5 104) (size 0.6) (drill 0.3) (layers "F.Cu" "B.Cu") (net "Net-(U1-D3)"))
 (segment (start 150 109.5) (end 144.5 104) (width 0.2) (layer "B.Cu") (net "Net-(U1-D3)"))
 (segment (start 159.5 109.5) (end 150 109.5) (width 0.2) (layer "B.Cu") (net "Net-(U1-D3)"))
 (segment (start 162.42 112.42) (end 159.5 109.5) (width 0.2) (layer "B.Cu") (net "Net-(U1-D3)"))
 (segment (start 177.12 112.42) (end 162.42 112.42) (width 0.2) (layer "B.Cu") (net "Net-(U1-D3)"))
 (segment (start 125.16 105.5) (end 130.5 100.16) (width 0.2) (layer "F.Cu") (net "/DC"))
 (segment (start 130.5 100.16) (end 138 100.16) (width 0.2) (layer "F.Cu") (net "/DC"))
 (segment (start 127.7 105.5) (end 130.5 102.7) (width 0.2) (layer "F.Cu") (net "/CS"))
 (segment (start 130.5 102.7) (end 138 102.7) (width 0.2) (layer "F.Cu") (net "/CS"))
 (segment (start 131.74 104) (end 136.76 104) (width 0.2) (layer "F.Cu") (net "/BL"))
 (segment (start 130.24 105.5) (end 130.74 105) (width 0.2) (layer "F.Cu") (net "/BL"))
 (segment (start 136.76 104) (end 138 105.24) (width 0.2) (layer "F.Cu") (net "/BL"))
 (segment (start 137.76 105) (end 138 105.24) (width 0.2) (layer "F.Cu") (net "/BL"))
 (segment (start 130.24 105.5) (end 131.74 104) (width 0.2) (layer "F.Cu") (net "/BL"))
 (segment (start 170.16 105.24) (end 153.24 105.24) (width 0.2) (layer "F.Cu") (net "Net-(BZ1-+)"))
 (segment (start 173.9 101.5) (end 170.16 105.24) (width 0.2) (layer "F.Cu") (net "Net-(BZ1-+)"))
 (segment (start 124.12 107) (end 146 107) (width 0.2) (layer "F.Cu") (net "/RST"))
 (segment (start 122.62 105.5) (end 124.12 107) (width 0.2) (layer "F.Cu") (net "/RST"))
 (segment (start 146 107) (end 149 104) (width 0.2) (layer "F.Cu") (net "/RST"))
 (via (at 149 104) (size 0.6) (drill 0.3) (layers "F.Cu" "B.Cu") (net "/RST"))
 (segment (start 149 104) (end 150.3 102.7) (width 0.2) (layer "B.Cu") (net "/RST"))
 (segment (start 150.3 102.7) (end 153.24 102.7) (width 0.2) (layer "B.Cu") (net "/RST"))
 (segment (start 117.54 105.5) (end 135.04 88) (width 0.2) (layer "B.Cu") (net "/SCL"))
 (segment (start 145 97.5) (end 147.66 100.16) (width 0.2) (layer "B.Cu") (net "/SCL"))
 (segment (start 145 91.5) (end 145 97.5) (width 0.2) (layer "B.Cu") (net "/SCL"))
 (segment (start 147.66 100.16) (end 153.24 100.16) (width 0.2) (layer "B.Cu") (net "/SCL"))
 (segment (start 135.04 88) (end 141.5 88) (width 0.2) (layer "B.Cu") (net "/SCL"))
 (segment (start 141.5 88) (end 145 91.5) (width 0.2) (layer "B.Cu") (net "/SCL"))
 (segment (start 120.08 105.5) (end 122.58 108) (width 0.2) (layer "F.Cu") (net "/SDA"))
 (segment (start 122.58 108) (end 147.5 108) (width 0.2) (layer "F.Cu") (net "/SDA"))
 (segment (start 152.38 97.62) (end 153.24 97.62) (width 0.2) (layer "F.Cu") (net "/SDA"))
 (segment (start 147.5 108) (end 150.5 105) (width 0.2) (layer "F.Cu") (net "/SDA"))
 (segment (start 150.5 105) (end 150.5 99.5) (width 0.2) (layer "F.Cu") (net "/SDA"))
 (segment (start 150.5 99.5) (end 152.38 97.62) (width 0.2) (layer "F.Cu") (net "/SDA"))
 (segment (start 115 105.5) (end 132.5 88) (width 0.2) (layer "F.Cu") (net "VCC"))
 (segment (start 143.08 95.08) (end 153.24 95.08) (width 0.2) (layer "F.Cu") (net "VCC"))
 (segment (start 138.5 88) (end 141 90.5) (width 0.2) (layer "F.Cu") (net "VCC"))
 (segment (start 132.5 88) (end 138.5 88) (width 0.2) (layer "F.Cu") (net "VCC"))
 (segment (start 141 93) (end 143.08 95.08) (width 0.2) (layer "F.Cu") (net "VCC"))
 (segment (start 141 90.5) (end 141 93) (width 0.2) (layer "F.Cu") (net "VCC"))
 (segment (start 153.24 90) (end 165.46 90) (width 0.2) (layer "F.Cu") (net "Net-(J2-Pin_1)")))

